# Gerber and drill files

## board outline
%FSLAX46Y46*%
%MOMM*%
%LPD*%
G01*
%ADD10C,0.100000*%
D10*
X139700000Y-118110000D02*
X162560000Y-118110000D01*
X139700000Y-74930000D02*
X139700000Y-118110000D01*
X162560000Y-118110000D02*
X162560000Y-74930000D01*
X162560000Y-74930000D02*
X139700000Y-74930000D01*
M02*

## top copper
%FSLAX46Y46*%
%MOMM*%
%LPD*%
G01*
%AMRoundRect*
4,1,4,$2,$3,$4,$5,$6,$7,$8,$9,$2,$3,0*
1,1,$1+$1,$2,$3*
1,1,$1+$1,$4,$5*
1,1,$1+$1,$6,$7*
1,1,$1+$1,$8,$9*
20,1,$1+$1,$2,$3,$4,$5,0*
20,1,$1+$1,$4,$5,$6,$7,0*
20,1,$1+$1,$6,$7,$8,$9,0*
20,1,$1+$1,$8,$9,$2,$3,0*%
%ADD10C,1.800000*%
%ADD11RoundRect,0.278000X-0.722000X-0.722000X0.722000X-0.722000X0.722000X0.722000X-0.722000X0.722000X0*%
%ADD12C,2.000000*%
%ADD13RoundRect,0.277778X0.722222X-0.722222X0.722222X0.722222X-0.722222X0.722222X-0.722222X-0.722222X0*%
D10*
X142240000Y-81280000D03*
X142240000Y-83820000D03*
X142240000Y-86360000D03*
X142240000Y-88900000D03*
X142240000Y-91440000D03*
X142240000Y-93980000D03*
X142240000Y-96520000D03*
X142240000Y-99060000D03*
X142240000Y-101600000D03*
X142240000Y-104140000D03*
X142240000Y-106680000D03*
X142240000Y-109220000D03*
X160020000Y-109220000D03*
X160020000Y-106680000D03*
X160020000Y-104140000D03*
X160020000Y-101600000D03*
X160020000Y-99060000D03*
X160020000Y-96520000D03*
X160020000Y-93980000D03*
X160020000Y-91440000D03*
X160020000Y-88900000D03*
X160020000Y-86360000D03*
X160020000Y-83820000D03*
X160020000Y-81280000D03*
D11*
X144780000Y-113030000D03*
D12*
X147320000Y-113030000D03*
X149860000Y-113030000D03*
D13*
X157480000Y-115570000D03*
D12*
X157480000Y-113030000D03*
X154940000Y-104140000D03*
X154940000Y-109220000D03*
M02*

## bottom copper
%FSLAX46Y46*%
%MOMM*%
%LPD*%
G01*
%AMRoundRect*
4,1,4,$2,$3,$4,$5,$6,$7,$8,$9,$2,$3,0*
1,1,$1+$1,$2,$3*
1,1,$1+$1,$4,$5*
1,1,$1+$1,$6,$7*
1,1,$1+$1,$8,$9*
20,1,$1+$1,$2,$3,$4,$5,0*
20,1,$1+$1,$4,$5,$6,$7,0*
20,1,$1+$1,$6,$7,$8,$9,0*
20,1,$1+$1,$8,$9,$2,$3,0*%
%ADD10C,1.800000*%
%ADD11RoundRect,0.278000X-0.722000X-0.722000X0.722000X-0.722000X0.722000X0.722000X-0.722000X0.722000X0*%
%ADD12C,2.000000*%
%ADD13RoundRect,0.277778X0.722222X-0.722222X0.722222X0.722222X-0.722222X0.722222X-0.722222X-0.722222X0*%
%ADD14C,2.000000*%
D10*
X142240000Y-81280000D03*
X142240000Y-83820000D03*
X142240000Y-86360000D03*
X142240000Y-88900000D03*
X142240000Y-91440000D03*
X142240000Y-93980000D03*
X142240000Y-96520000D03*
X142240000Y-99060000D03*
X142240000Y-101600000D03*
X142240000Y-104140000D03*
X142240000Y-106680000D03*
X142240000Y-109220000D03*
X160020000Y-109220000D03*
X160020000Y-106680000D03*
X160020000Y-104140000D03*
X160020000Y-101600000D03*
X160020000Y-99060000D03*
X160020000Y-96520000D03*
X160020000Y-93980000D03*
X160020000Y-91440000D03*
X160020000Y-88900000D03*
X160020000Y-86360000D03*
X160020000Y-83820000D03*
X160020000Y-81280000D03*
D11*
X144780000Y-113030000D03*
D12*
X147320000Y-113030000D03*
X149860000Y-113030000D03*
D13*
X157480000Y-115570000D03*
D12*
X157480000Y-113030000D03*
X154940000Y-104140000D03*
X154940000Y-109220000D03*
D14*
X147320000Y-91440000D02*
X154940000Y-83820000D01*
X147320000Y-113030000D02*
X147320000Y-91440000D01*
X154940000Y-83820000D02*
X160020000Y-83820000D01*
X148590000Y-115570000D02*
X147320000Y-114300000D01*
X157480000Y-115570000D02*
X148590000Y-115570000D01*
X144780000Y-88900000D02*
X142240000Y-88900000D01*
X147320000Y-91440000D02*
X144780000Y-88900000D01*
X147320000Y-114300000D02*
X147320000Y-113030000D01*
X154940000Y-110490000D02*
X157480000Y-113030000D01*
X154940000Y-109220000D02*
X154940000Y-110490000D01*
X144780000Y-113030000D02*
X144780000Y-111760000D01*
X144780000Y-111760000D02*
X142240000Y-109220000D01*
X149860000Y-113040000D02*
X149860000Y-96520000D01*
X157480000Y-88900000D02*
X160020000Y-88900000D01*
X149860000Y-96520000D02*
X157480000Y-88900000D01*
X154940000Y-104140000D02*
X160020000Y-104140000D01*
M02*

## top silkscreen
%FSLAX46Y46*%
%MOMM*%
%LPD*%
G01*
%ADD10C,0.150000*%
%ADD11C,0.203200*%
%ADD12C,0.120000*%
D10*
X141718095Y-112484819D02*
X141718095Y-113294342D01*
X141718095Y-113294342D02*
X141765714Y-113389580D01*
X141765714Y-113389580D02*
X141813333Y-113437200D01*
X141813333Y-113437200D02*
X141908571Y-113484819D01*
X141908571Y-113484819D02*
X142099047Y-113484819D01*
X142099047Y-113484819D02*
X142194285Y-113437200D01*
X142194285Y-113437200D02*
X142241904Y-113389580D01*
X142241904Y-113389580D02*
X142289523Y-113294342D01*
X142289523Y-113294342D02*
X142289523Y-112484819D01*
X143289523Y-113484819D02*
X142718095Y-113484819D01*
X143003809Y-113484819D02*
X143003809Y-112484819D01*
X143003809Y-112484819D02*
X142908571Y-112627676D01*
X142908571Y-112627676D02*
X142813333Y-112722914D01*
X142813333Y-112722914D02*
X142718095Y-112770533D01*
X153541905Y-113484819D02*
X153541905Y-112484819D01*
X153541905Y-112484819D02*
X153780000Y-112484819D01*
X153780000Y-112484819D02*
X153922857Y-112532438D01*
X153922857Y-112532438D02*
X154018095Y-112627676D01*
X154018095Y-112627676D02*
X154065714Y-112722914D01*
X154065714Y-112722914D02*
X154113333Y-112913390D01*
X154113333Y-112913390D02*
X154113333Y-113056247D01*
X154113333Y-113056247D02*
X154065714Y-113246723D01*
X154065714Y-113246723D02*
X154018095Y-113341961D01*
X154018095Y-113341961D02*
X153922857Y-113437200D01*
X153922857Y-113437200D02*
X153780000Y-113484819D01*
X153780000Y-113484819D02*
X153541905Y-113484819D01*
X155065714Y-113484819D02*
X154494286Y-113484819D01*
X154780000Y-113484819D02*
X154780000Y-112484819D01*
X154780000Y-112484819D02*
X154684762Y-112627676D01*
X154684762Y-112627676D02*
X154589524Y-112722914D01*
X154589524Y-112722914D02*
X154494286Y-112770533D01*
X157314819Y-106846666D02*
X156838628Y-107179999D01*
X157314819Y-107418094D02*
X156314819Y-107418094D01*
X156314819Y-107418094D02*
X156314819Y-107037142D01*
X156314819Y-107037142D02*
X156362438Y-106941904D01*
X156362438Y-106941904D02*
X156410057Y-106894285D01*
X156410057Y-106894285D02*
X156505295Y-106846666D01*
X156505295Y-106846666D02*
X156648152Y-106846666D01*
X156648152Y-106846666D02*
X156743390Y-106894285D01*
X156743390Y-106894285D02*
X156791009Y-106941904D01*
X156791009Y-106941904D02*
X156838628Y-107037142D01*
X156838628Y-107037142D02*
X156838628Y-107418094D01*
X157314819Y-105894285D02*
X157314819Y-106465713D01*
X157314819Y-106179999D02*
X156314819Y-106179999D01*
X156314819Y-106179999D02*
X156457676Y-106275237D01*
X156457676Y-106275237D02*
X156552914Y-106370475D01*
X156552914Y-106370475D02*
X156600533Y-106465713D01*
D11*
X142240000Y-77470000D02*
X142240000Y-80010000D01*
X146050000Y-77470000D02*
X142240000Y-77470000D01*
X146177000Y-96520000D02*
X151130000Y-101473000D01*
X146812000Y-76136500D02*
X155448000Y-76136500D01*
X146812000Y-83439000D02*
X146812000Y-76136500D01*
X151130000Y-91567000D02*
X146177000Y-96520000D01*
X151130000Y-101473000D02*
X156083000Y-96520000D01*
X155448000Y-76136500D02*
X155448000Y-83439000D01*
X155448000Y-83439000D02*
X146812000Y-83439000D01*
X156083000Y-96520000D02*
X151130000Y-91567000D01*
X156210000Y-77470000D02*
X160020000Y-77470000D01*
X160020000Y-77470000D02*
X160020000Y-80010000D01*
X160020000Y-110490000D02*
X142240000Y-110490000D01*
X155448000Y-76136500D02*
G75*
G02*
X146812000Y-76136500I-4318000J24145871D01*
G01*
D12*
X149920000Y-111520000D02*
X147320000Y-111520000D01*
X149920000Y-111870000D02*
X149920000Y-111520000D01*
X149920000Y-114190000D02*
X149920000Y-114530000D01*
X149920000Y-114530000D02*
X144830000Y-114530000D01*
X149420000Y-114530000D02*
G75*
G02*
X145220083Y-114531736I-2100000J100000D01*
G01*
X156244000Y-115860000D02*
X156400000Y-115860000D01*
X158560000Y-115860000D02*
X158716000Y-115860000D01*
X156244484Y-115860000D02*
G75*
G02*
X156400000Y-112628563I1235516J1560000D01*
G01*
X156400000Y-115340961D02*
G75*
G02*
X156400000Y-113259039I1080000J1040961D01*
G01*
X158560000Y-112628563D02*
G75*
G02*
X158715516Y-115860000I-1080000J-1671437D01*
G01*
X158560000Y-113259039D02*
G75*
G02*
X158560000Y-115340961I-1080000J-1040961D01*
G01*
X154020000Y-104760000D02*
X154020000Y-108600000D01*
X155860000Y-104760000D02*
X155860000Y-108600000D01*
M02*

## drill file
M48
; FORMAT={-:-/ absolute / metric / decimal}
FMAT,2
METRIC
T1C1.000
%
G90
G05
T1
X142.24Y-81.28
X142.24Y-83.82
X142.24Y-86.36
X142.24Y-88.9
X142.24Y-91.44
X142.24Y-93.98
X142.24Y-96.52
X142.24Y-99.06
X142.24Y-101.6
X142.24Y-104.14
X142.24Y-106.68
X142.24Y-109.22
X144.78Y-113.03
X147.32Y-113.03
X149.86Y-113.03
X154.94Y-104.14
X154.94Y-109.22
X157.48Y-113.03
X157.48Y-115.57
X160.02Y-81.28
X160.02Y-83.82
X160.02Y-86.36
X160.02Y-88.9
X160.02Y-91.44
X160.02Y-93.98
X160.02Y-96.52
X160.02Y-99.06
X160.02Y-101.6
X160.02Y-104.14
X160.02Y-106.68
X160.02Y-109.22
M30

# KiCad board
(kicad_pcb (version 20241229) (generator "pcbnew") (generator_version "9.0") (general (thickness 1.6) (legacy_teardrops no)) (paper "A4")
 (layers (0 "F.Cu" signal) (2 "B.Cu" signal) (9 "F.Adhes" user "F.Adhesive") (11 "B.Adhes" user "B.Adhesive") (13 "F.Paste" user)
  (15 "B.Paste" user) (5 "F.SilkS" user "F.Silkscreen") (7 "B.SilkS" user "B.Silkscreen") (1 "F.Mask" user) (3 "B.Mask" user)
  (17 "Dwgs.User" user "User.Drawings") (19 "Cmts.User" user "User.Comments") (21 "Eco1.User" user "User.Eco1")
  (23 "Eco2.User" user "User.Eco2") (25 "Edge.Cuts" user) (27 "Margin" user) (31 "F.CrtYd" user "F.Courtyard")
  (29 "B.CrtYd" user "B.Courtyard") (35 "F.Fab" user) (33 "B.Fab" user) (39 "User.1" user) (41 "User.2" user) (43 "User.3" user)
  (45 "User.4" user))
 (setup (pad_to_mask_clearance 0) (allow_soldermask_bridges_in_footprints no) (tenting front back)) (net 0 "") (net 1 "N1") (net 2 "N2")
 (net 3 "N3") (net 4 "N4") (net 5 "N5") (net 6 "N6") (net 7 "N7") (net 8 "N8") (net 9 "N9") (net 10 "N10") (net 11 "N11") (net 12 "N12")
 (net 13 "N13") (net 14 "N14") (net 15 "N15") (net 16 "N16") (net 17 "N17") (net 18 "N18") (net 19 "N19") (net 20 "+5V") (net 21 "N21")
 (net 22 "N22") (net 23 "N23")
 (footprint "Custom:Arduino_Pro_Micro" (layer "F.Cu") (at 151.13 93.98)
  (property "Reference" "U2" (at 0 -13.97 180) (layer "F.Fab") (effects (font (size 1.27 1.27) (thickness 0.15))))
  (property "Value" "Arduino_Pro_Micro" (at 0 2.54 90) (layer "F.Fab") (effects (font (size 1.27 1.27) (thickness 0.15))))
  (fp_line (start -8.89 -16.51) (end -8.89 -13.97) (stroke (width 0.2032) (type solid)) (layer "F.SilkS"))
  (fp_line (start -5.08 -16.51) (end -8.89 -16.51) (stroke (width 0.2032) (type solid)) (layer "F.SilkS"))
  (fp_line (start -4.953 2.54) (end 0 7.493) (stroke (width 0.2032) (type solid)) (layer "F.SilkS"))
  (fp_line (start -4.318 -17.8435) (end 4.318 -17.8435) (stroke (width 0.2032) (type solid)) (layer "F.SilkS"))
  (fp_line (start -4.318 -10.541) (end -4.318 -17.8435) (stroke (width 0.2032) (type solid)) (layer "F.SilkS"))
  (fp_line (start 0 -2.413) (end -4.953 2.54) (stroke (width 0.2032) (type solid)) (layer "F.SilkS"))
  (fp_line (start 0 7.493) (end 4.953 2.54) (stroke (width 0.2032) (type solid)) (layer "F.SilkS"))
  (fp_line (start 4.318 -17.8435) (end 4.318 -10.541) (stroke (width 0.2032) (type solid)) (layer "F.SilkS"))
  (fp_line (start 4.318 -10.541) (end -4.318 -10.541) (stroke (width 0.2032) (type solid)) (layer "F.SilkS"))
  (fp_line (start 4.953 2.54) (end 0 -2.413) (stroke (width 0.2032) (type solid)) (layer "F.SilkS"))
  (fp_line (start 5.08 -16.51) (end 8.89 -16.51) (stroke (width 0.2032) (type solid)) (layer "F.SilkS"))
  (fp_line (start 8.89 -16.51) (end 8.89 -13.97) (stroke (width 0.2032) (type solid)) (layer "F.SilkS"))
  (fp_line (start 8.89 16.51) (end -8.89 16.51) (stroke (width 0.2032) (type solid)) (layer "F.SilkS"))
  (fp_arc (start 4.318 -17.8435) (mid 0 -17.460445) (end -4.318 -17.8435) (stroke (width 0.2032) (type solid)) (layer "F.SilkS"))
  (pad "1" thru_hole circle (at -8.89 -12.7) (size 1.8 1.8) (drill 1) (layers "*.Cu" "*.Mask") (remove_unused_layers no) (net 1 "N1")
   (thermal_bridge_angle 0))
  (pad "2" thru_hole circle (at -8.89 -10.16) (size 1.8 1.8) (drill 1) (layers "*.Cu" "*.Mask") (remove_unused_layers no) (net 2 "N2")
   (thermal_bridge_angle 0))
  (pad "3" thru_hole circle (at -8.89 -7.62) (size 1.8 1.8) (drill 1) (layers "*.Cu" "*.Mask") (remove_unused_layers no) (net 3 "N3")
   (thermal_bridge_angle 0))
  (pad "4" thru_hole circle (at -8.89 -5.08) (size 1.8 1.8) (drill 1) (layers "*.Cu" "*.Mask") (remove_unused_layers no) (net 3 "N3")
   (thermal_bridge_angle 0))
  (pad "5" thru_hole circle (at -8.89 -2.54) (size 1.8 1.8) (drill 1) (layers "*.Cu" "*.Mask") (remove_unused_layers no) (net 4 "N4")
   (thermal_bridge_angle 0))
  (pad "6" thru_hole circle (at -8.89 0) (size 1.8 1.8) (drill 1) (layers "*.Cu" "*.Mask") (remove_unused_layers no) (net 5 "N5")
   (thermal_bridge_angle 0))
  (pad "7" thru_hole circle (at -8.89 2.54) (size 1.8 1.8) (drill 1) (layers "*.Cu" "*.Mask") (remove_unused_layers no) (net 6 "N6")
   (thermal_bridge_angle 0))
  (pad "8" thru_hole circle (at -8.89 5.08) (size 1.8 1.8) (drill 1) (layers "*.Cu" "*.Mask") (remove_unused_layers no) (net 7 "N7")
   (thermal_bridge_angle 0))
  (pad "9" thru_hole circle (at -8.89 7.62) (size 1.8 1.8) (drill 1) (layers "*.Cu" "*.Mask") (remove_unused_layers no) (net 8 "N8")
   (thermal_bridge_angle 0))
  (pad "10" thru_hole circle (at -8.89 10.16) (size 1.8 1.8) (drill 1) (layers "*.Cu" "*.Mask") (remove_unused_layers no) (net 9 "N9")
   (thermal_bridge_angle 0))
  (pad "11" thru_hole circle (at -8.89 12.7) (size 1.8 1.8) (drill 1) (layers "*.Cu" "*.Mask") (remove_unused_layers no) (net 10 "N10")
   (thermal_bridge_angle 0))
  (pad "12" thru_hole circle (at -8.89 15.24) (size 1.8 1.8) (drill 1) (layers "*.Cu" "*.Mask") (remove_unused_layers no) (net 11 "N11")
   (thermal_bridge_angle 0))
  (pad "13" thru_hole circle (at 8.89 15.24) (size 1.8 1.8) (drill 1) (layers "*.Cu" "*.Mask") (remove_unused_layers no) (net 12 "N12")
   (thermal_bridge_angle 0))
  (pad "14" thru_hole circle (at 8.89 12.7) (size 1.8 1.8) (drill 1) (layers "*.Cu" "*.Mask") (remove_unused_layers no) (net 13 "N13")
   (thermal_bridge_angle 0))
  (pad "15" thru_hole circle (at 8.89 10.16) (size 1.8 1.8) (drill 1) (layers "*.Cu" "*.Mask") (remove_unused_layers no) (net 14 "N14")
   (thermal_bridge_angle 0))
  (pad "16" thru_hole circle (at 8.89 7.62) (size 1.8 1.8) (drill 1) (layers "*.Cu" "*.Mask") (remove_unused_layers no) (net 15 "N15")
   (thermal_bridge_angle 0))
  (pad "17" thru_hole circle (at 8.89 5.08) (size 1.8 1.8) (drill 1) (layers "*.Cu" "*.Mask") (remove_unused_layers no) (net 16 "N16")
   (thermal_bridge_angle 0))
  (pad "18" thru_hole circle (at 8.89 2.54) (size 1.8 1.8) (drill 1) (layers "*.Cu" "*.Mask") (remove_unused_layers no) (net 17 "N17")
   (thermal_bridge_angle 0))
  (pad "19" thru_hole circle (at 8.89 0) (size 1.8 1.8) (drill 1) (layers "*.Cu" "*.Mask") (remove_unused_layers no) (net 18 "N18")
   (thermal_bridge_angle 0))
  (pad "20" thru_hole circle (at 8.89 -2.54) (size 1.8 1.8) (drill 1) (layers "*.Cu" "*.Mask") (remove_unused_layers no) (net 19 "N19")
   (thermal_bridge_angle 0))
  (pad "21" thru_hole circle (at 8.89 -5.08) (size 1.8 1.8) (drill 1) (layers "*.Cu" "*.Mask") (remove_unused_layers no) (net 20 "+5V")
   (thermal_bridge_angle 0))
  (pad "22" thru_hole circle (at 8.89 -7.62) (size 1.8 1.8) (drill 1) (layers "*.Cu" "*.Mask") (remove_unused_layers no) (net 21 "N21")
   (thermal_bridge_angle 0))
  (pad "23" thru_hole circle (at 8.89 -10.16) (size 1.8 1.8) (drill 1) (layers "*.Cu" "*.Mask") (remove_unused_layers no) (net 3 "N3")
   (thermal_bridge_angle 0))
  (pad "24" thru_hole circle (at 8.89 -12.7) (size 1.8 1.8) (drill 1) (layers "*.Cu" "*.Mask") (remove_unused_layers no) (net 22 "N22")
   (thermal_bridge_angle 0)))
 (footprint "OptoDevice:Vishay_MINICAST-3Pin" (layer "F.Cu") (at 144.78 113.03)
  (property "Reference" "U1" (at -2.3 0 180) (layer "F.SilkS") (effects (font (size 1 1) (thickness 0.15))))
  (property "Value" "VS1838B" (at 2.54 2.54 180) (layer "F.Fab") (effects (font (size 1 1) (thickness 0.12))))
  (fp_line (start 5.14 -1.51) (end 2.54 -1.51) (stroke (width 0.12) (type solid)) (layer "F.SilkS"))
  (fp_line (start 5.14 -1.16) (end 5.14 -1.51) (stroke (width 0.12) (type solid)) (layer "F.SilkS"))
  (fp_line (start 5.14 1.16) (end 5.14 1.5) (stroke (width 0.12) (type solid)) (layer "F.SilkS"))
  (fp_line (start 5.14 1.5) (end 0.05 1.5) (stroke (width 0.12) (type solid)) (layer "F.SilkS"))
  (fp_arc (start 4.64 1.5) (mid 2.540869 3.502379) (end 0.440083 1.501736) (stroke (width 0.12) (type solid)) (layer "F.SilkS"))
  (pad "1" thru_hole roundrect (at 0 0) (size 2 2) (drill 1) (layers "*.Cu" "*.Mask") (remove_unused_layers no) (roundrect_rratio 0.139)
   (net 11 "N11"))
  (pad "2" thru_hole circle (at 2.54 0) (size 2 2) (drill 1) (layers "*.Cu" "*.Mask") (remove_unused_layers no) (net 3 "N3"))
  (pad "3" thru_hole circle (at 5.08 0) (size 2 2) (drill 1) (layers "*.Cu" "*.Mask") (remove_unused_layers no) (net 20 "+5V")))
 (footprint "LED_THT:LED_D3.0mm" (layer "F.Cu") (at 157.48 115.57 90)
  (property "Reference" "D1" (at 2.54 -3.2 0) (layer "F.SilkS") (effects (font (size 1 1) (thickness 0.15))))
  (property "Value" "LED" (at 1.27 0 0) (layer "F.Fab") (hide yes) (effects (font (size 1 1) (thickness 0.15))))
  (fp_line (start -0.29 -1.236) (end -0.29 -1.08) (stroke (width 0.12) (type solid)) (layer "F.SilkS"))
  (fp_line (start -0.29 1.08) (end -0.29 1.236) (stroke (width 0.12) (type solid)) (layer "F.SilkS"))
  (fp_arc (start -0.29 -1.235516) (mid 1.36566 -1.987699) (end 2.941437 -1.08) (stroke (width 0.12) (type solid)) (layer "F.SilkS"))
  (fp_arc (start 0.229039 -1.08) (mid 1.27 -1.5) (end 2.310961 -1.08) (stroke (width 0.12) (type solid)) (layer "F.SilkS"))
  (fp_arc (start 2.941437 1.08) (mid 1.36566 1.987699) (end -0.29 1.235516) (stroke (width 0.12) (type solid)) (layer "F.SilkS"))
  (fp_arc (start 2.310961 1.08) (mid 1.27 1.5) (end 0.229039 1.08) (stroke (width 0.12) (type solid)) (layer "F.SilkS"))
  (pad "1" thru_hole roundrect (at 0 0 90) (size 2 2) (drill 1) (layers "*.Cu" "*.Mask") (remove_unused_layers no)
   (roundrect_rratio 0.1388888889) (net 3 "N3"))
  (pad "2" thru_hole circle (at 2.54 0 90) (size 2 2) (drill 1) (layers "*.Cu" "*.Mask") (remove_unused_layers no) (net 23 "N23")))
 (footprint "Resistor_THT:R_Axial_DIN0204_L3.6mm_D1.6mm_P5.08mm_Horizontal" (layer "F.Cu") (at 154.94 104.14 -90)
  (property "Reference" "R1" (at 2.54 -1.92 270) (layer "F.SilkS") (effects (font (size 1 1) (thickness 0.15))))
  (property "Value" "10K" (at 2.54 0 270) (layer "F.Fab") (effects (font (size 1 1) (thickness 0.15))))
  (fp_line (start 0.62 0.92) (end 4.46 0.92) (stroke (width 0.12) (type solid)) (layer "F.SilkS"))
  (fp_line (start 0.62 -0.92) (end 4.46 -0.92) (stroke (width 0.12) (type solid)) (layer "F.SilkS"))
  (pad "1" thru_hole circle (at 0 0 270) (size 2 2) (drill 1) (layers "*.Cu" "*.Mask") (remove_unused_layers no) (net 14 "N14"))
  (pad "2" thru_hole circle (at 5.08 0 270) (size 2 2) (drill 1) (layers "*.Cu" "*.Mask") (remove_unused_layers no) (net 23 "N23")))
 (gr_line (start 139.7 118.11) (end 162.56 118.11) (stroke (width 0.1) (type solid)) (layer "Edge.Cuts"))
 (gr_line (start 139.7 74.93) (end 139.7 118.11) (stroke (width 0.1) (type default)) (layer "Edge.Cuts"))
 (gr_line (start 162.56 118.11) (end 162.56 74.93) (stroke (width 0.1) (type default)) (layer "Edge.Cuts"))
 (gr_line (start 162.56 74.93) (end 139.7 74.93) (stroke (width 0.1) (type solid)) (layer "Edge.Cuts"))
 (segment (start 147.32 91.44) (end 154.94 83.82) (width 2) (layer "B.Cu") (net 3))
 (segment (start 147.32 113.03) (end 147.32 91.44) (width 2) (layer "B.Cu") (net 3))
 (segment (start 154.94 83.82) (end 160.02 83.82) (width 2) (layer "B.Cu") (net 3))
 (segment (start 148.59 115.57) (end 147.32 114.3) (width 2) (layer "B.Cu") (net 3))
 (segment (start 157.48 115.57) (end 148.59 115.57) (width 2) (layer "B.Cu") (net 3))
 (segment (start 144.78 88.9) (end 142.24 88.9) (width 2) (layer "B.Cu") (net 3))
 (segment (start 147.32 91.44) (end 144.78 88.9) (width 2) (layer "B.Cu") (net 3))
 (segment (start 147.32 114.3) (end 147.32 113.03) (width 2) (layer "B.Cu") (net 3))
 (segment (start 154.94 110.49) (end 157.48 113.03) (width 2) (layer "B.Cu") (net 23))
 (segment (start 154.94 109.22) (end 154.94 110.49) (width 2) (layer "B.Cu") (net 23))
 (segment (start 144.78 113.03) (end 144.78 111.76) (width 2) (layer "B.Cu") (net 11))
 (segment (start 144.78 111.76) (end 142.24 109.22) (width 2) (layer "B.Cu") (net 11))
 (segment (start 149.86 113.04) (end 149.86 96.52) (width 2) (layer "B.Cu") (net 20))
 (segment (start 157.48 88.9) (end 160.02 88.9) (width 2) (layer "B.Cu") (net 20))
 (segment (start 149.86 96.52) (end 157.48 88.9) (width 2) (layer "B.Cu") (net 20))
 (segment (start 154.94 104.14) (end 160.02 104.14) (width 2) (layer "B.Cu") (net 14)))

